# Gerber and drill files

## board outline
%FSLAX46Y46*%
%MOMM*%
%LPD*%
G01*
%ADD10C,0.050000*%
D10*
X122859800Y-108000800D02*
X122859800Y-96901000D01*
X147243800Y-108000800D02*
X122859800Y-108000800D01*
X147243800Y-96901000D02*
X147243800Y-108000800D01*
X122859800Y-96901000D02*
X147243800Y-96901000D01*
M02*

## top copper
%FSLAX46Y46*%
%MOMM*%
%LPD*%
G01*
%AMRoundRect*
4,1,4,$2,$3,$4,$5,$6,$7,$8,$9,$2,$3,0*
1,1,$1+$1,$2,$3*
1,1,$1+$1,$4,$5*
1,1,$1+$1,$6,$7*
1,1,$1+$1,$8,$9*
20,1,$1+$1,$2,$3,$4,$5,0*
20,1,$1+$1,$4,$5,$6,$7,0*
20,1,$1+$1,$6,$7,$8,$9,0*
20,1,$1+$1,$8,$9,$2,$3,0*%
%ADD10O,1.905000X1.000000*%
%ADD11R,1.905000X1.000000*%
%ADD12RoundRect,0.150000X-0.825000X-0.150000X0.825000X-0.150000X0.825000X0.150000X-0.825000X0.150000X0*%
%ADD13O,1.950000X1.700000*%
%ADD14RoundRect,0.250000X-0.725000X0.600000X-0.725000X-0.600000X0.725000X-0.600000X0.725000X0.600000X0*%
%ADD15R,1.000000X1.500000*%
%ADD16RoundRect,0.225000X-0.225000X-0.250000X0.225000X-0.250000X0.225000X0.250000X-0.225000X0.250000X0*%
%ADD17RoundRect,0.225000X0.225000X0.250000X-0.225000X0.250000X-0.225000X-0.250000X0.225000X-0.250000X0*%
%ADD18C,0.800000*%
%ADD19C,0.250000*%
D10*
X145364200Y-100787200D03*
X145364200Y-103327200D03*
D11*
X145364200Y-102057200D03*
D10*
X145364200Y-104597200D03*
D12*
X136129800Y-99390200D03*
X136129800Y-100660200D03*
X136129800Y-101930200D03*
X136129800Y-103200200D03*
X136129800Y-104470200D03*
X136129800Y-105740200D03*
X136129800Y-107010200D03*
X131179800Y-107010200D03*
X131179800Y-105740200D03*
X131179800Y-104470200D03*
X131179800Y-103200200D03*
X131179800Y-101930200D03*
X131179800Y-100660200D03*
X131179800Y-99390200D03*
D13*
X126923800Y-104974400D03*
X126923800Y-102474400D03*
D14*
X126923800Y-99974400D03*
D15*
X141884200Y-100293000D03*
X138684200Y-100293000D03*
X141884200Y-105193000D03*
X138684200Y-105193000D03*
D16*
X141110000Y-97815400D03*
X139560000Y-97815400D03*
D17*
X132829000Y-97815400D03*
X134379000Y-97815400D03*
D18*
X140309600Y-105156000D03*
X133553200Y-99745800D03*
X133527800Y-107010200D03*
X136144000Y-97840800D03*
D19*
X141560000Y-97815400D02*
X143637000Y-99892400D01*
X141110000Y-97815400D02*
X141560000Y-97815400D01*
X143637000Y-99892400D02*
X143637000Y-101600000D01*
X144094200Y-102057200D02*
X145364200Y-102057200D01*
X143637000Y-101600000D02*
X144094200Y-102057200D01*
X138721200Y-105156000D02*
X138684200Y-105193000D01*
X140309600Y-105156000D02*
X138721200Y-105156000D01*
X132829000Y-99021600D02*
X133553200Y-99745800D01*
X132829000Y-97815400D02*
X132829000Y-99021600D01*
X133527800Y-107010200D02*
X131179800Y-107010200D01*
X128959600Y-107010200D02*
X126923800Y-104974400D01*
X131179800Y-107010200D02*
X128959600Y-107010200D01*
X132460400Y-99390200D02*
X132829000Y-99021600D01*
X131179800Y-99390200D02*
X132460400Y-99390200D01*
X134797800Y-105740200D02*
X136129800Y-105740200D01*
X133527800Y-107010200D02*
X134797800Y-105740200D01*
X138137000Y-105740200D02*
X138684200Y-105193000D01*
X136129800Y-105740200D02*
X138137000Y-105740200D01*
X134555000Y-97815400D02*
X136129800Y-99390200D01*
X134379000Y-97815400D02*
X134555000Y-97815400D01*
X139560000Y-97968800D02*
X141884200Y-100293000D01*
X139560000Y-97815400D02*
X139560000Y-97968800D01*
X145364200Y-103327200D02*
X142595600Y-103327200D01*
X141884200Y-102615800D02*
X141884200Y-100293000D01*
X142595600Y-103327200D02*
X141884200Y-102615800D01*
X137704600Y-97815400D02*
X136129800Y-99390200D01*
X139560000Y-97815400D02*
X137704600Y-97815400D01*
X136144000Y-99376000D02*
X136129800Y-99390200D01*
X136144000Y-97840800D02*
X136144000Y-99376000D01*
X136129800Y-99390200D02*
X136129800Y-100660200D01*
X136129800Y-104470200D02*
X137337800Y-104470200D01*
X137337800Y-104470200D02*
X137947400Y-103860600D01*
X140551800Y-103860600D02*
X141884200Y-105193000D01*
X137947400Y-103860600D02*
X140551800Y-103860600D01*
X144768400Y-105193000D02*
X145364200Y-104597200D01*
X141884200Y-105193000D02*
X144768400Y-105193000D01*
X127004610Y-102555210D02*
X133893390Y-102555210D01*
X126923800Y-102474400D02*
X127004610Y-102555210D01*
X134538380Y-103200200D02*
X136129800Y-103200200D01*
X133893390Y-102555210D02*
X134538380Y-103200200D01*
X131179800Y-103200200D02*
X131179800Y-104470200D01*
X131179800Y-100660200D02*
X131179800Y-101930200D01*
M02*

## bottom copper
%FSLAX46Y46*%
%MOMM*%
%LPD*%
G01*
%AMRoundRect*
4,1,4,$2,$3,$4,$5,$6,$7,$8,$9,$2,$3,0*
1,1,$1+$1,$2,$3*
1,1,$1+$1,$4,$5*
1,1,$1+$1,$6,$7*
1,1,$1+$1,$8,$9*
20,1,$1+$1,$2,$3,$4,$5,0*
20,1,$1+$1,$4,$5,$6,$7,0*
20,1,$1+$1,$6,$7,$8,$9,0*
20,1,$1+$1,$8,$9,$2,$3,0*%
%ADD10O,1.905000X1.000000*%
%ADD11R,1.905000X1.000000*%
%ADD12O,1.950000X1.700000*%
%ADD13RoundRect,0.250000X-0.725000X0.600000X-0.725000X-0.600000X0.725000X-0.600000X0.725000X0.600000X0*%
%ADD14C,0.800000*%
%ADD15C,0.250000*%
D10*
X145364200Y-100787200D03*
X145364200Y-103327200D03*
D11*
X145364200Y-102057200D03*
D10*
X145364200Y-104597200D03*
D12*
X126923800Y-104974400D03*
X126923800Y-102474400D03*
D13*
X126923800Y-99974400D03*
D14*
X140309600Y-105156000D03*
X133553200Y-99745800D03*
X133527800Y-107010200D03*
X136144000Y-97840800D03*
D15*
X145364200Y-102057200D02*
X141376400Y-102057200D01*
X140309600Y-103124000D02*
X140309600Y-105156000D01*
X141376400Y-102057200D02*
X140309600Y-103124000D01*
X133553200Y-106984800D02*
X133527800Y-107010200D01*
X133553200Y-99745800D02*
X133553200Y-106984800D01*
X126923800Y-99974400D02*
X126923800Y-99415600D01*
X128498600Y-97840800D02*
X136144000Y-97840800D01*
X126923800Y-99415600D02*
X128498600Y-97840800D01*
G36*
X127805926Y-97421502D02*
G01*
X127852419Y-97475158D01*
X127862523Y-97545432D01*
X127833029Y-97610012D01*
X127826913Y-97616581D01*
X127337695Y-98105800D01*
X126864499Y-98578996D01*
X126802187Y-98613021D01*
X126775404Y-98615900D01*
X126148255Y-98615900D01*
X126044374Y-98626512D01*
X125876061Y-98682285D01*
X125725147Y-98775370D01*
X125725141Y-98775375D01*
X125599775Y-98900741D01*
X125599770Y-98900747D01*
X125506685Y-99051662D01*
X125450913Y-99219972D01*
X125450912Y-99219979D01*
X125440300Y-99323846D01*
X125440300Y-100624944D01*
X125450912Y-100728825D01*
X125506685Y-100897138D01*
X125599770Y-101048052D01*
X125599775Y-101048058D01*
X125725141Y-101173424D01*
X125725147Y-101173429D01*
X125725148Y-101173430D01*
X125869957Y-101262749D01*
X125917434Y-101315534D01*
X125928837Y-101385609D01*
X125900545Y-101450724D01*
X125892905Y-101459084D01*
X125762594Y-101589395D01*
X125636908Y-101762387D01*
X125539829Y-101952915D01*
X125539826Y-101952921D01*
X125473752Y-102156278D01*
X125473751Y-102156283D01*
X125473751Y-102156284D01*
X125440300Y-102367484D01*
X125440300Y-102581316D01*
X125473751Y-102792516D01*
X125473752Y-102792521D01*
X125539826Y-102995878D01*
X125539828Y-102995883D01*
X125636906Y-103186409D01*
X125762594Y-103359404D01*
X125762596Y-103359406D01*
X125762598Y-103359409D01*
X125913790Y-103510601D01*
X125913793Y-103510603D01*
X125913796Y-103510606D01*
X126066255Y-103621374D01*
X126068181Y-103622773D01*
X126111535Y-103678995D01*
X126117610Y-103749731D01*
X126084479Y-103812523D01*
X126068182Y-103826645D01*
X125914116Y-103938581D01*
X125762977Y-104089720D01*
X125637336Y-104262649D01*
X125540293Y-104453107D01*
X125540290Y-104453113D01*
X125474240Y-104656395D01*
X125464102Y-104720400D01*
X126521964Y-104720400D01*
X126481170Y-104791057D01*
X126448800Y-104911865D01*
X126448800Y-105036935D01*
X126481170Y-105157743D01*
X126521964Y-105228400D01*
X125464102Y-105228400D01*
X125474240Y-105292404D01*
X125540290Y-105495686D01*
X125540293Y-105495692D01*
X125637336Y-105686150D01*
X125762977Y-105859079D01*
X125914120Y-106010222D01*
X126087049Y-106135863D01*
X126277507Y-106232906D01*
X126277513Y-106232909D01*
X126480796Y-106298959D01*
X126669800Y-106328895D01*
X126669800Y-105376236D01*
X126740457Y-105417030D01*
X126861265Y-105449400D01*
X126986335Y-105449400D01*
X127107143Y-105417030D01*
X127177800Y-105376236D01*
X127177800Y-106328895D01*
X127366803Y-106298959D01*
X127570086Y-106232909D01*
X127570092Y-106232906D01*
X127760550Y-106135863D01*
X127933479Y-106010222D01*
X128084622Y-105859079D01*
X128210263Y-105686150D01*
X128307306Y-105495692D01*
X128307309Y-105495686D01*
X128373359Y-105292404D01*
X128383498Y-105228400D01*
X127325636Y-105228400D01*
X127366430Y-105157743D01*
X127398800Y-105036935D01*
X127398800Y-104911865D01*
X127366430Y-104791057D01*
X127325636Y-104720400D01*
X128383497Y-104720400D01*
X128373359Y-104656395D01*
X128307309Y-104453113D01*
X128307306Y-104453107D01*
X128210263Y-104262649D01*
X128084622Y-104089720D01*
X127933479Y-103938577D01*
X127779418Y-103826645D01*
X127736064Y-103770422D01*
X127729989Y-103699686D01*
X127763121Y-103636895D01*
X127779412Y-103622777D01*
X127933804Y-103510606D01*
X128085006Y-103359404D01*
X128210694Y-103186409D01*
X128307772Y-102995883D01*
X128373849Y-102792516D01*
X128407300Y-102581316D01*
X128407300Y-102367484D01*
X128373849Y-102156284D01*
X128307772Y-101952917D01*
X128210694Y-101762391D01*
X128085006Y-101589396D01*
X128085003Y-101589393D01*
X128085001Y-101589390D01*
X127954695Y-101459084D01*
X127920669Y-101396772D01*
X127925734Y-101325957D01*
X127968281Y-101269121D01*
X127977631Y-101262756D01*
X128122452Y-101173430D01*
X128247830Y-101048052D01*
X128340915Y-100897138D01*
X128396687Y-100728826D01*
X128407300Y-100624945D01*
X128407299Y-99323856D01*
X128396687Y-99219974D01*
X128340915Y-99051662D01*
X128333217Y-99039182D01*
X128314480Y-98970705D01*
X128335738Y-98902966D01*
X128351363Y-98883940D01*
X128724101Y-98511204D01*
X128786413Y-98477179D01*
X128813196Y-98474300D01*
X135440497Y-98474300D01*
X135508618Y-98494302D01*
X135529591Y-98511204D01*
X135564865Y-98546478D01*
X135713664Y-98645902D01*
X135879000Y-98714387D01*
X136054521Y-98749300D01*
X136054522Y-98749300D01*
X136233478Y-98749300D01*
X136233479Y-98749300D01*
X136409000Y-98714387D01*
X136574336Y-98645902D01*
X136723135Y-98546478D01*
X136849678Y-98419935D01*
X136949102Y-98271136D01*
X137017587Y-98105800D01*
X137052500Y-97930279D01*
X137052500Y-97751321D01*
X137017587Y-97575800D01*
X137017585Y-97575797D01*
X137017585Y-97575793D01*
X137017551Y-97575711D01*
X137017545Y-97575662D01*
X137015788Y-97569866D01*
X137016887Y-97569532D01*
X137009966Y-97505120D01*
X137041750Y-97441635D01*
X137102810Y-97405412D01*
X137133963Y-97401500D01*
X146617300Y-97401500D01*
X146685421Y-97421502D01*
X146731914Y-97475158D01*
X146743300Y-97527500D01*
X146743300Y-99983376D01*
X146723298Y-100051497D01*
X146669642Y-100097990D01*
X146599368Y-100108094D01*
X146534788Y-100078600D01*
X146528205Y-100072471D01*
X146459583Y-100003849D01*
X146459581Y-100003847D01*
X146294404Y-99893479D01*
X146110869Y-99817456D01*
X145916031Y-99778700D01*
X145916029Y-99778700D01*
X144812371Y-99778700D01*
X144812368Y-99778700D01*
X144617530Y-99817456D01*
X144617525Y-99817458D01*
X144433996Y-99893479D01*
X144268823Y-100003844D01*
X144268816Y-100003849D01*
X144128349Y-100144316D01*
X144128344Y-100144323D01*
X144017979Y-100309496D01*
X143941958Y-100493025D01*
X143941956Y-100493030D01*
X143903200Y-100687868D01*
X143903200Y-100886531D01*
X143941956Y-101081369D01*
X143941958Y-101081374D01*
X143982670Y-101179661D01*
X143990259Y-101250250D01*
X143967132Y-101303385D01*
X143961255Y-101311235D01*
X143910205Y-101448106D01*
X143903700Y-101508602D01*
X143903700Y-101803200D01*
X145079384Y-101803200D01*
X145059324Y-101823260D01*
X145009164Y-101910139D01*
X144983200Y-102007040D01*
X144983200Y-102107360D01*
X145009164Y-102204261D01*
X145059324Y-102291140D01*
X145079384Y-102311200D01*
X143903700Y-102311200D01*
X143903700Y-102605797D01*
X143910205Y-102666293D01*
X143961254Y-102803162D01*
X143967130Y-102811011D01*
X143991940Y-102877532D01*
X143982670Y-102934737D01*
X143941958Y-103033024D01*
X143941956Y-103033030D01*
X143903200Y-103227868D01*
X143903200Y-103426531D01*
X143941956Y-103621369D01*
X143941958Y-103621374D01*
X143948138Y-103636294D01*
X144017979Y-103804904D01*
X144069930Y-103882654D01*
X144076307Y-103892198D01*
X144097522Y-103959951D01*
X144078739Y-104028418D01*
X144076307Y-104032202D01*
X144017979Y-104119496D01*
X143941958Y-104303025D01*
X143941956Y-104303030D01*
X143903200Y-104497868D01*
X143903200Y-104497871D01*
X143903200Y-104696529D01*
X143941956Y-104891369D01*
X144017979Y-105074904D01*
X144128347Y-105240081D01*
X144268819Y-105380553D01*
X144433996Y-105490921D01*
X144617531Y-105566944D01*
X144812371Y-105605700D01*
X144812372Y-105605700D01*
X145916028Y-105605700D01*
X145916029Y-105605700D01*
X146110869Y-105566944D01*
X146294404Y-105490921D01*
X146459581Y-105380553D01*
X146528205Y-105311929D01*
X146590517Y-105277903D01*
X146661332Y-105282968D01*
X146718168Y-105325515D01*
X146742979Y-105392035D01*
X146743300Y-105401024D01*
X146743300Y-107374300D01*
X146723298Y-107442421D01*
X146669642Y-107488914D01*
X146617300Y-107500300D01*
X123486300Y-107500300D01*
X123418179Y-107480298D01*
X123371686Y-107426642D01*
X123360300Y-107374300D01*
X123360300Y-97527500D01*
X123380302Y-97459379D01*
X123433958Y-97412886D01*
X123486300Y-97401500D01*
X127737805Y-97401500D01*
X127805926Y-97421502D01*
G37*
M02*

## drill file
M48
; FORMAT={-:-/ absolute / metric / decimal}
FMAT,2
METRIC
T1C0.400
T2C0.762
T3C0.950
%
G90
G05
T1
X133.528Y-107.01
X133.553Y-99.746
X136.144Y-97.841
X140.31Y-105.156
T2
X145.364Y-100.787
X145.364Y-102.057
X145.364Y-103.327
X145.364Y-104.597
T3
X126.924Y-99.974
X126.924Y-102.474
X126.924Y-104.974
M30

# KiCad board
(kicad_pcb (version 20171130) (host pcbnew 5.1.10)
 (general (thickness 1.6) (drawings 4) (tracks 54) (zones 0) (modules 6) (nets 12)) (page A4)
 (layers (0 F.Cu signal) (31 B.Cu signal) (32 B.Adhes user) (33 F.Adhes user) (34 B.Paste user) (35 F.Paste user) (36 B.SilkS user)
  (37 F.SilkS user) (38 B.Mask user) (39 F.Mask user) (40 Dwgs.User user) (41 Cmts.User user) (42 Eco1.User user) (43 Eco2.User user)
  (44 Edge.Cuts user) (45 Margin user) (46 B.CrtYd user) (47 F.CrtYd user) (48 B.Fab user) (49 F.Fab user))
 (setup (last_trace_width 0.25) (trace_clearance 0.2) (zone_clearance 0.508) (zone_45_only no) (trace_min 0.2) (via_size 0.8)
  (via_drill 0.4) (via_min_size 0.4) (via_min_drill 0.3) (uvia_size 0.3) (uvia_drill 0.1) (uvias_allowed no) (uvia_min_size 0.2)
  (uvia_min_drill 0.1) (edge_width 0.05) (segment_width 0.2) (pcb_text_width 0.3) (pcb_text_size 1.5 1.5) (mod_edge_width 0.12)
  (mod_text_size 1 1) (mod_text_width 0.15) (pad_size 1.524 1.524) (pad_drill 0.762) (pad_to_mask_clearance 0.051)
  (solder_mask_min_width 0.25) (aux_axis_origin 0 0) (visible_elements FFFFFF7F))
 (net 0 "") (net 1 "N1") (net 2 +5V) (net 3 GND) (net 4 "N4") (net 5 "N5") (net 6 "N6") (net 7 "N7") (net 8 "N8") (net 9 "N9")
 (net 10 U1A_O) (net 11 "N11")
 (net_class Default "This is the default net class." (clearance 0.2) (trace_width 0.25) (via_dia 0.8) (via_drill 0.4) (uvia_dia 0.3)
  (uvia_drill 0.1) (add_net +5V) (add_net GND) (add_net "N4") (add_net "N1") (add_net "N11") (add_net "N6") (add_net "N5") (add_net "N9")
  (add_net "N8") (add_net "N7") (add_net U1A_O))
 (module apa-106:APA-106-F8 (layer F.Cu) (at 145.3642 102.6922 90)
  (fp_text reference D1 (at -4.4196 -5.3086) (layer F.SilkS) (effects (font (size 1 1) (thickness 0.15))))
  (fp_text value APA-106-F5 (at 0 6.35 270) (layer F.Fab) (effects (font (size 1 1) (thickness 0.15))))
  (pad 4 thru_hole oval (at 1.905 0 180) (size 1.905 1) (drill 0.762) (layers *.Cu *.Mask) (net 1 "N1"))
  (pad 2 thru_hole oval (at -0.635 0 180) (size 1.905 1) (drill 0.762) (layers *.Cu *.Mask) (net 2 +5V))
  (pad 3 thru_hole rect (at 0.635 0 180) (size 1.905 1) (drill 0.762) (layers *.Cu *.Mask) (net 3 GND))
  (pad 1 thru_hole oval (at -1.905 0 180) (size 1.905 1) (drill 0.762) (layers *.Cu *.Mask) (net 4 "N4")))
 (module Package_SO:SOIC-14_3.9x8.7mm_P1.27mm (layer F.Cu) (at 133.6548 103.2002)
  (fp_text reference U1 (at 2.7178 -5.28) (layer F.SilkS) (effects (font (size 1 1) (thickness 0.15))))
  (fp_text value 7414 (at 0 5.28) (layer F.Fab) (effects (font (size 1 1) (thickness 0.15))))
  (pad 14 smd roundrect (at 2.475 -3.81) (size 1.95 0.6) (layers F.Cu F.Paste F.Mask) (roundrect_rratio 0.25) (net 2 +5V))
  (pad 13 smd roundrect (at 2.475 -2.54) (size 1.95 0.6) (layers F.Cu F.Paste F.Mask) (roundrect_rratio 0.25) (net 2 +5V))
  (pad 12 smd roundrect (at 2.475 -1.27) (size 1.95 0.6) (layers F.Cu F.Paste F.Mask) (roundrect_rratio 0.25) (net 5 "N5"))
  (pad 11 smd roundrect (at 2.475 0) (size 1.95 0.6) (layers F.Cu F.Paste F.Mask) (roundrect_rratio 0.25) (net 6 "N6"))
  (pad 10 smd roundrect (at 2.475 1.27) (size 1.95 0.6) (layers F.Cu F.Paste F.Mask) (roundrect_rratio 0.25) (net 4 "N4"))
  (pad 9 smd roundrect (at 2.475 2.54) (size 1.95 0.6) (layers F.Cu F.Paste F.Mask) (roundrect_rratio 0.25) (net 3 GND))
  (pad 8 smd roundrect (at 2.475 3.81) (size 1.95 0.6) (layers F.Cu F.Paste F.Mask) (roundrect_rratio 0.25) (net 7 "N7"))
  (pad 7 smd roundrect (at -2.475 3.81) (size 1.95 0.6) (layers F.Cu F.Paste F.Mask) (roundrect_rratio 0.25) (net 3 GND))
  (pad 6 smd roundrect (at -2.475 2.54) (size 1.95 0.6) (layers F.Cu F.Paste F.Mask) (roundrect_rratio 0.25) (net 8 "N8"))
  (pad 5 smd roundrect (at -2.475 1.27) (size 1.95 0.6) (layers F.Cu F.Paste F.Mask) (roundrect_rratio 0.25) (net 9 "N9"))
  (pad 4 smd roundrect (at -2.475 0) (size 1.95 0.6) (layers F.Cu F.Paste F.Mask) (roundrect_rratio 0.25) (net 9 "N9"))
  (pad 3 smd roundrect (at -2.475 -1.27) (size 1.95 0.6) (layers F.Cu F.Paste F.Mask) (roundrect_rratio 0.25) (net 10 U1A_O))
  (pad 2 smd roundrect (at -2.475 -2.54) (size 1.95 0.6) (layers F.Cu F.Paste F.Mask) (roundrect_rratio 0.25) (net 10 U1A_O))
  (pad 1 smd roundrect (at -2.475 -3.81) (size 1.95 0.6) (layers F.Cu F.Paste F.Mask) (roundrect_rratio 0.25) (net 3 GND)))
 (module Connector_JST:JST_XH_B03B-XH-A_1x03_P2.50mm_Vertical (layer F.Cu) (at 126.9238 99.9744 270)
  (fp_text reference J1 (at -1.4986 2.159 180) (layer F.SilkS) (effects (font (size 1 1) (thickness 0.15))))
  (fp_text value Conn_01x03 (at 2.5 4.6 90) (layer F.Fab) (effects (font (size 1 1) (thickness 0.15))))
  (pad 3 thru_hole oval (at 5 0 270) (size 1.7 1.95) (drill 0.95) (layers *.Cu *.Mask) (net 3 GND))
  (pad 2 thru_hole oval (at 2.5 0 270) (size 1.7 1.95) (drill 0.95) (layers *.Cu *.Mask) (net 6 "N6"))
  (pad 1 thru_hole roundrect (at 0 0 270) (size 1.7 1.95) (drill 0.95) (layers *.Cu *.Mask) (roundrect_rratio 0.147059) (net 2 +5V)))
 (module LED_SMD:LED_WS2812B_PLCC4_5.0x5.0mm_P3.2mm (layer F.Cu) (at 140.2842 102.743 270)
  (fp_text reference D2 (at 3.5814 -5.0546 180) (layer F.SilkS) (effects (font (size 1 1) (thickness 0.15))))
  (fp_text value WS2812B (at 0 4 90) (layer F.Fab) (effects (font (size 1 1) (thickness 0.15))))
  (pad 1 smd rect (at -2.45 -1.6 270) (size 1.5 1) (layers F.Cu F.Paste F.Mask) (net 2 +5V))
  (pad 2 smd rect (at -2.45 1.6 270) (size 1.5 1) (layers F.Cu F.Paste F.Mask) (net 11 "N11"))
  (pad 4 smd rect (at 2.45 -1.6 270) (size 1.5 1) (layers F.Cu F.Paste F.Mask) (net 4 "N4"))
  (pad 3 smd rect (at 2.45 1.6 270) (size 1.5 1) (layers F.Cu F.Paste F.Mask) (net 3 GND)))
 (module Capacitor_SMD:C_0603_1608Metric (layer F.Cu) (at 140.335 97.8154)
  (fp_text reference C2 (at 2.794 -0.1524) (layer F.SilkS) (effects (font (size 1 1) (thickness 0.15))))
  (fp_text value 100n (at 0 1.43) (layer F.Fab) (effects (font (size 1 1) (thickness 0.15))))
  (pad 2 smd roundrect (at 0.775 0) (size 0.9 0.95) (layers F.Cu F.Paste F.Mask) (roundrect_rratio 0.25) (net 3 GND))
  (pad 1 smd roundrect (at -0.775 0) (size 0.9 0.95) (layers F.Cu F.Paste F.Mask) (roundrect_rratio 0.25) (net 2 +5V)))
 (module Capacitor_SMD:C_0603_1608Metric (layer F.Cu) (at 133.604 97.8154 180)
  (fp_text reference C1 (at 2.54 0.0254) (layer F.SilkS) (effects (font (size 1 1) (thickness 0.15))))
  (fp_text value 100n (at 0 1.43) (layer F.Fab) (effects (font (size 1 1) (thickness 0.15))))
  (pad 2 smd roundrect (at 0.775 0 180) (size 0.9 0.95) (layers F.Cu F.Paste F.Mask) (roundrect_rratio 0.25) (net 3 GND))
  (pad 1 smd roundrect (at -0.775 0 180) (size 0.9 0.95) (layers F.Cu F.Paste F.Mask) (roundrect_rratio 0.25) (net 2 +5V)))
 (gr_line (start 122.8598 108.0008) (end 122.8598 96.901) (layer Edge.Cuts) (width 0.05))
 (gr_line (start 147.2438 108.0008) (end 122.8598 108.0008) (layer Edge.Cuts) (width 0.05))
 (gr_line (start 147.2438 96.901) (end 147.2438 108.0008) (layer Edge.Cuts) (width 0.05))
 (gr_line (start 122.8598 96.901) (end 147.2438 96.901) (layer Edge.Cuts) (width 0.05))
 (segment (start 141.56 97.8154) (end 143.637 99.8924) (width 0.25) (layer F.Cu) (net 3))
 (segment (start 141.11 97.8154) (end 141.56 97.8154) (width 0.25) (layer F.Cu) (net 3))
 (segment (start 143.637 99.8924) (end 143.637 101.6) (width 0.25) (layer F.Cu) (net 3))
 (segment (start 144.0942 102.0572) (end 145.3642 102.0572) (width 0.25) (layer F.Cu) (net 3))
 (segment (start 143.637 101.6) (end 144.0942 102.0572) (width 0.25) (layer F.Cu) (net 3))
 (segment (start 145.3642 102.0572) (end 141.3764 102.0572) (width 0.25) (layer B.Cu) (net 3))
 (via (at 140.3096 105.156) (size 0.8) (drill 0.4) (layers F.Cu B.Cu) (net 3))
 (segment (start 140.3096 103.124) (end 140.3096 105.156) (width 0.25) (layer B.Cu) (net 3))
 (segment (start 141.3764 102.0572) (end 140.3096 103.124) (width 0.25) (layer B.Cu) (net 3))
 (segment (start 138.7212 105.156) (end 138.6842 105.193) (width 0.25) (layer F.Cu) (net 3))
 (segment (start 140.3096 105.156) (end 138.7212 105.156) (width 0.25) (layer F.Cu) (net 3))
 (via (at 133.5532 99.7458) (size 0.8) (drill 0.4) (layers F.Cu B.Cu) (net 3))
 (segment (start 132.829 99.0216) (end 133.5532 99.7458) (width 0.25) (layer F.Cu) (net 3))
 (segment (start 132.829 97.8154) (end 132.829 99.0216) (width 0.25) (layer F.Cu) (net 3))
 (segment (start 133.5532 106.9848) (end 133.5278 107.0102) (width 0.25) (layer B.Cu) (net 3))
 (via (at 133.5278 107.0102) (size 0.8) (drill 0.4) (layers F.Cu B.Cu) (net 3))
 (segment (start 133.5532 99.7458) (end 133.5532 106.9848) (width 0.25) (layer B.Cu) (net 3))
 (segment (start 133.5278 107.0102) (end 131.1798 107.0102) (width 0.25) (layer F.Cu) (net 3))
 (segment (start 128.9596 107.0102) (end 126.9238 104.9744) (width 0.25) (layer F.Cu) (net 3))
 (segment (start 131.1798 107.0102) (end 128.9596 107.0102) (width 0.25) (layer F.Cu) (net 3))
 (segment (start 132.4604 99.3902) (end 132.829 99.0216) (width 0.25) (layer F.Cu) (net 3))
 (segment (start 131.1798 99.3902) (end 132.4604 99.3902) (width 0.25) (layer F.Cu) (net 3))
 (segment (start 134.7978 105.7402) (end 136.1298 105.7402) (width 0.25) (layer F.Cu) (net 3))
 (segment (start 133.5278 107.0102) (end 134.7978 105.7402) (width 0.25) (layer F.Cu) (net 3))
 (segment (start 138.137 105.7402) (end 138.6842 105.193) (width 0.25) (layer F.Cu) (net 3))
 (segment (start 136.1298 105.7402) (end 138.137 105.7402) (width 0.25) (layer F.Cu) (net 3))
 (segment (start 134.555 97.8154) (end 136.1298 99.3902) (width 0.25) (layer F.Cu) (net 2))
 (segment (start 134.379 97.8154) (end 134.555 97.8154) (width 0.25) (layer F.Cu) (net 2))
 (segment (start 139.56 97.9688) (end 141.8842 100.293) (width 0.25) (layer F.Cu) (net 2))
 (segment (start 139.56 97.8154) (end 139.56 97.9688) (width 0.25) (layer F.Cu) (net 2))
 (segment (start 145.3642 103.3272) (end 142.5956 103.3272) (width 0.25) (layer F.Cu) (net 2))
 (segment (start 141.8842 102.6158) (end 141.8842 100.293) (width 0.25) (layer F.Cu) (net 2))
 (segment (start 142.5956 103.3272) (end 141.8842 102.6158) (width 0.25) (layer F.Cu) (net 2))
 (segment (start 137.7046 97.8154) (end 136.1298 99.3902) (width 0.25) (layer F.Cu) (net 2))
 (segment (start 139.56 97.8154) (end 137.7046 97.8154) (width 0.25) (layer F.Cu) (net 2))
 (segment (start 126.9238 99.9744) (end 126.9238 99.4156) (width 0.25) (layer B.Cu) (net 2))
 (via (at 136.144 97.8408) (size 0.8) (drill 0.4) (layers F.Cu B.Cu) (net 2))
 (segment (start 128.4986 97.8408) (end 136.144 97.8408) (width 0.25) (layer B.Cu) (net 2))
 (segment (start 126.9238 99.4156) (end 128.4986 97.8408) (width 0.25) (layer B.Cu) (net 2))
 (segment (start 136.144 99.376) (end 136.1298 99.3902) (width 0.25) (layer F.Cu) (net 2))
 (segment (start 136.144 97.8408) (end 136.144 99.376) (width 0.25) (layer F.Cu) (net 2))
 (segment (start 136.1298 99.3902) (end 136.1298 100.6602) (width 0.25) (layer F.Cu) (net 2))
 (segment (start 136.1298 104.4702) (end 137.3378 104.4702) (width 0.25) (layer F.Cu) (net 4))
 (segment (start 137.3378 104.4702) (end 137.9474 103.8606) (width 0.25) (layer F.Cu) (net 4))
 (segment (start 140.5518 103.8606) (end 141.8842 105.193) (width 0.25) (layer F.Cu) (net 4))
 (segment (start 137.9474 103.8606) (end 140.5518 103.8606) (width 0.25) (layer F.Cu) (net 4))
 (segment (start 144.7684 105.193) (end 145.3642 104.5972) (width 0.25) (layer F.Cu) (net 4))
 (segment (start 141.8842 105.193) (end 144.7684 105.193) (width 0.25) (layer F.Cu) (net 4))
 (segment (start 127.00461 102.55521) (end 133.89339 102.55521) (width 0.25) (layer F.Cu) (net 6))
 (segment (start 126.9238 102.4744) (end 127.00461 102.55521) (width 0.25) (layer F.Cu) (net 6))
 (segment (start 134.53838 103.2002) (end 136.1298 103.2002) (width 0.25) (layer F.Cu) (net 6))
 (segment (start 133.89339 102.55521) (end 134.53838 103.2002) (width 0.25) (layer F.Cu) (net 6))
 (segment (start 131.1798 103.2002) (end 131.1798 104.4702) (width 0.25) (layer F.Cu) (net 9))
 (segment (start 131.1798 100.6602) (end 131.1798 101.9302) (width 0.25) (layer F.Cu) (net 10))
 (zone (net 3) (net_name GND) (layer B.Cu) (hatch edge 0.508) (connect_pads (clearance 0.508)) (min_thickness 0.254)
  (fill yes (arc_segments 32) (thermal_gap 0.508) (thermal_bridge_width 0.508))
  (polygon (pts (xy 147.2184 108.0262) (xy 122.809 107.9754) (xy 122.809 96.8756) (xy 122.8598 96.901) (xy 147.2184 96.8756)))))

